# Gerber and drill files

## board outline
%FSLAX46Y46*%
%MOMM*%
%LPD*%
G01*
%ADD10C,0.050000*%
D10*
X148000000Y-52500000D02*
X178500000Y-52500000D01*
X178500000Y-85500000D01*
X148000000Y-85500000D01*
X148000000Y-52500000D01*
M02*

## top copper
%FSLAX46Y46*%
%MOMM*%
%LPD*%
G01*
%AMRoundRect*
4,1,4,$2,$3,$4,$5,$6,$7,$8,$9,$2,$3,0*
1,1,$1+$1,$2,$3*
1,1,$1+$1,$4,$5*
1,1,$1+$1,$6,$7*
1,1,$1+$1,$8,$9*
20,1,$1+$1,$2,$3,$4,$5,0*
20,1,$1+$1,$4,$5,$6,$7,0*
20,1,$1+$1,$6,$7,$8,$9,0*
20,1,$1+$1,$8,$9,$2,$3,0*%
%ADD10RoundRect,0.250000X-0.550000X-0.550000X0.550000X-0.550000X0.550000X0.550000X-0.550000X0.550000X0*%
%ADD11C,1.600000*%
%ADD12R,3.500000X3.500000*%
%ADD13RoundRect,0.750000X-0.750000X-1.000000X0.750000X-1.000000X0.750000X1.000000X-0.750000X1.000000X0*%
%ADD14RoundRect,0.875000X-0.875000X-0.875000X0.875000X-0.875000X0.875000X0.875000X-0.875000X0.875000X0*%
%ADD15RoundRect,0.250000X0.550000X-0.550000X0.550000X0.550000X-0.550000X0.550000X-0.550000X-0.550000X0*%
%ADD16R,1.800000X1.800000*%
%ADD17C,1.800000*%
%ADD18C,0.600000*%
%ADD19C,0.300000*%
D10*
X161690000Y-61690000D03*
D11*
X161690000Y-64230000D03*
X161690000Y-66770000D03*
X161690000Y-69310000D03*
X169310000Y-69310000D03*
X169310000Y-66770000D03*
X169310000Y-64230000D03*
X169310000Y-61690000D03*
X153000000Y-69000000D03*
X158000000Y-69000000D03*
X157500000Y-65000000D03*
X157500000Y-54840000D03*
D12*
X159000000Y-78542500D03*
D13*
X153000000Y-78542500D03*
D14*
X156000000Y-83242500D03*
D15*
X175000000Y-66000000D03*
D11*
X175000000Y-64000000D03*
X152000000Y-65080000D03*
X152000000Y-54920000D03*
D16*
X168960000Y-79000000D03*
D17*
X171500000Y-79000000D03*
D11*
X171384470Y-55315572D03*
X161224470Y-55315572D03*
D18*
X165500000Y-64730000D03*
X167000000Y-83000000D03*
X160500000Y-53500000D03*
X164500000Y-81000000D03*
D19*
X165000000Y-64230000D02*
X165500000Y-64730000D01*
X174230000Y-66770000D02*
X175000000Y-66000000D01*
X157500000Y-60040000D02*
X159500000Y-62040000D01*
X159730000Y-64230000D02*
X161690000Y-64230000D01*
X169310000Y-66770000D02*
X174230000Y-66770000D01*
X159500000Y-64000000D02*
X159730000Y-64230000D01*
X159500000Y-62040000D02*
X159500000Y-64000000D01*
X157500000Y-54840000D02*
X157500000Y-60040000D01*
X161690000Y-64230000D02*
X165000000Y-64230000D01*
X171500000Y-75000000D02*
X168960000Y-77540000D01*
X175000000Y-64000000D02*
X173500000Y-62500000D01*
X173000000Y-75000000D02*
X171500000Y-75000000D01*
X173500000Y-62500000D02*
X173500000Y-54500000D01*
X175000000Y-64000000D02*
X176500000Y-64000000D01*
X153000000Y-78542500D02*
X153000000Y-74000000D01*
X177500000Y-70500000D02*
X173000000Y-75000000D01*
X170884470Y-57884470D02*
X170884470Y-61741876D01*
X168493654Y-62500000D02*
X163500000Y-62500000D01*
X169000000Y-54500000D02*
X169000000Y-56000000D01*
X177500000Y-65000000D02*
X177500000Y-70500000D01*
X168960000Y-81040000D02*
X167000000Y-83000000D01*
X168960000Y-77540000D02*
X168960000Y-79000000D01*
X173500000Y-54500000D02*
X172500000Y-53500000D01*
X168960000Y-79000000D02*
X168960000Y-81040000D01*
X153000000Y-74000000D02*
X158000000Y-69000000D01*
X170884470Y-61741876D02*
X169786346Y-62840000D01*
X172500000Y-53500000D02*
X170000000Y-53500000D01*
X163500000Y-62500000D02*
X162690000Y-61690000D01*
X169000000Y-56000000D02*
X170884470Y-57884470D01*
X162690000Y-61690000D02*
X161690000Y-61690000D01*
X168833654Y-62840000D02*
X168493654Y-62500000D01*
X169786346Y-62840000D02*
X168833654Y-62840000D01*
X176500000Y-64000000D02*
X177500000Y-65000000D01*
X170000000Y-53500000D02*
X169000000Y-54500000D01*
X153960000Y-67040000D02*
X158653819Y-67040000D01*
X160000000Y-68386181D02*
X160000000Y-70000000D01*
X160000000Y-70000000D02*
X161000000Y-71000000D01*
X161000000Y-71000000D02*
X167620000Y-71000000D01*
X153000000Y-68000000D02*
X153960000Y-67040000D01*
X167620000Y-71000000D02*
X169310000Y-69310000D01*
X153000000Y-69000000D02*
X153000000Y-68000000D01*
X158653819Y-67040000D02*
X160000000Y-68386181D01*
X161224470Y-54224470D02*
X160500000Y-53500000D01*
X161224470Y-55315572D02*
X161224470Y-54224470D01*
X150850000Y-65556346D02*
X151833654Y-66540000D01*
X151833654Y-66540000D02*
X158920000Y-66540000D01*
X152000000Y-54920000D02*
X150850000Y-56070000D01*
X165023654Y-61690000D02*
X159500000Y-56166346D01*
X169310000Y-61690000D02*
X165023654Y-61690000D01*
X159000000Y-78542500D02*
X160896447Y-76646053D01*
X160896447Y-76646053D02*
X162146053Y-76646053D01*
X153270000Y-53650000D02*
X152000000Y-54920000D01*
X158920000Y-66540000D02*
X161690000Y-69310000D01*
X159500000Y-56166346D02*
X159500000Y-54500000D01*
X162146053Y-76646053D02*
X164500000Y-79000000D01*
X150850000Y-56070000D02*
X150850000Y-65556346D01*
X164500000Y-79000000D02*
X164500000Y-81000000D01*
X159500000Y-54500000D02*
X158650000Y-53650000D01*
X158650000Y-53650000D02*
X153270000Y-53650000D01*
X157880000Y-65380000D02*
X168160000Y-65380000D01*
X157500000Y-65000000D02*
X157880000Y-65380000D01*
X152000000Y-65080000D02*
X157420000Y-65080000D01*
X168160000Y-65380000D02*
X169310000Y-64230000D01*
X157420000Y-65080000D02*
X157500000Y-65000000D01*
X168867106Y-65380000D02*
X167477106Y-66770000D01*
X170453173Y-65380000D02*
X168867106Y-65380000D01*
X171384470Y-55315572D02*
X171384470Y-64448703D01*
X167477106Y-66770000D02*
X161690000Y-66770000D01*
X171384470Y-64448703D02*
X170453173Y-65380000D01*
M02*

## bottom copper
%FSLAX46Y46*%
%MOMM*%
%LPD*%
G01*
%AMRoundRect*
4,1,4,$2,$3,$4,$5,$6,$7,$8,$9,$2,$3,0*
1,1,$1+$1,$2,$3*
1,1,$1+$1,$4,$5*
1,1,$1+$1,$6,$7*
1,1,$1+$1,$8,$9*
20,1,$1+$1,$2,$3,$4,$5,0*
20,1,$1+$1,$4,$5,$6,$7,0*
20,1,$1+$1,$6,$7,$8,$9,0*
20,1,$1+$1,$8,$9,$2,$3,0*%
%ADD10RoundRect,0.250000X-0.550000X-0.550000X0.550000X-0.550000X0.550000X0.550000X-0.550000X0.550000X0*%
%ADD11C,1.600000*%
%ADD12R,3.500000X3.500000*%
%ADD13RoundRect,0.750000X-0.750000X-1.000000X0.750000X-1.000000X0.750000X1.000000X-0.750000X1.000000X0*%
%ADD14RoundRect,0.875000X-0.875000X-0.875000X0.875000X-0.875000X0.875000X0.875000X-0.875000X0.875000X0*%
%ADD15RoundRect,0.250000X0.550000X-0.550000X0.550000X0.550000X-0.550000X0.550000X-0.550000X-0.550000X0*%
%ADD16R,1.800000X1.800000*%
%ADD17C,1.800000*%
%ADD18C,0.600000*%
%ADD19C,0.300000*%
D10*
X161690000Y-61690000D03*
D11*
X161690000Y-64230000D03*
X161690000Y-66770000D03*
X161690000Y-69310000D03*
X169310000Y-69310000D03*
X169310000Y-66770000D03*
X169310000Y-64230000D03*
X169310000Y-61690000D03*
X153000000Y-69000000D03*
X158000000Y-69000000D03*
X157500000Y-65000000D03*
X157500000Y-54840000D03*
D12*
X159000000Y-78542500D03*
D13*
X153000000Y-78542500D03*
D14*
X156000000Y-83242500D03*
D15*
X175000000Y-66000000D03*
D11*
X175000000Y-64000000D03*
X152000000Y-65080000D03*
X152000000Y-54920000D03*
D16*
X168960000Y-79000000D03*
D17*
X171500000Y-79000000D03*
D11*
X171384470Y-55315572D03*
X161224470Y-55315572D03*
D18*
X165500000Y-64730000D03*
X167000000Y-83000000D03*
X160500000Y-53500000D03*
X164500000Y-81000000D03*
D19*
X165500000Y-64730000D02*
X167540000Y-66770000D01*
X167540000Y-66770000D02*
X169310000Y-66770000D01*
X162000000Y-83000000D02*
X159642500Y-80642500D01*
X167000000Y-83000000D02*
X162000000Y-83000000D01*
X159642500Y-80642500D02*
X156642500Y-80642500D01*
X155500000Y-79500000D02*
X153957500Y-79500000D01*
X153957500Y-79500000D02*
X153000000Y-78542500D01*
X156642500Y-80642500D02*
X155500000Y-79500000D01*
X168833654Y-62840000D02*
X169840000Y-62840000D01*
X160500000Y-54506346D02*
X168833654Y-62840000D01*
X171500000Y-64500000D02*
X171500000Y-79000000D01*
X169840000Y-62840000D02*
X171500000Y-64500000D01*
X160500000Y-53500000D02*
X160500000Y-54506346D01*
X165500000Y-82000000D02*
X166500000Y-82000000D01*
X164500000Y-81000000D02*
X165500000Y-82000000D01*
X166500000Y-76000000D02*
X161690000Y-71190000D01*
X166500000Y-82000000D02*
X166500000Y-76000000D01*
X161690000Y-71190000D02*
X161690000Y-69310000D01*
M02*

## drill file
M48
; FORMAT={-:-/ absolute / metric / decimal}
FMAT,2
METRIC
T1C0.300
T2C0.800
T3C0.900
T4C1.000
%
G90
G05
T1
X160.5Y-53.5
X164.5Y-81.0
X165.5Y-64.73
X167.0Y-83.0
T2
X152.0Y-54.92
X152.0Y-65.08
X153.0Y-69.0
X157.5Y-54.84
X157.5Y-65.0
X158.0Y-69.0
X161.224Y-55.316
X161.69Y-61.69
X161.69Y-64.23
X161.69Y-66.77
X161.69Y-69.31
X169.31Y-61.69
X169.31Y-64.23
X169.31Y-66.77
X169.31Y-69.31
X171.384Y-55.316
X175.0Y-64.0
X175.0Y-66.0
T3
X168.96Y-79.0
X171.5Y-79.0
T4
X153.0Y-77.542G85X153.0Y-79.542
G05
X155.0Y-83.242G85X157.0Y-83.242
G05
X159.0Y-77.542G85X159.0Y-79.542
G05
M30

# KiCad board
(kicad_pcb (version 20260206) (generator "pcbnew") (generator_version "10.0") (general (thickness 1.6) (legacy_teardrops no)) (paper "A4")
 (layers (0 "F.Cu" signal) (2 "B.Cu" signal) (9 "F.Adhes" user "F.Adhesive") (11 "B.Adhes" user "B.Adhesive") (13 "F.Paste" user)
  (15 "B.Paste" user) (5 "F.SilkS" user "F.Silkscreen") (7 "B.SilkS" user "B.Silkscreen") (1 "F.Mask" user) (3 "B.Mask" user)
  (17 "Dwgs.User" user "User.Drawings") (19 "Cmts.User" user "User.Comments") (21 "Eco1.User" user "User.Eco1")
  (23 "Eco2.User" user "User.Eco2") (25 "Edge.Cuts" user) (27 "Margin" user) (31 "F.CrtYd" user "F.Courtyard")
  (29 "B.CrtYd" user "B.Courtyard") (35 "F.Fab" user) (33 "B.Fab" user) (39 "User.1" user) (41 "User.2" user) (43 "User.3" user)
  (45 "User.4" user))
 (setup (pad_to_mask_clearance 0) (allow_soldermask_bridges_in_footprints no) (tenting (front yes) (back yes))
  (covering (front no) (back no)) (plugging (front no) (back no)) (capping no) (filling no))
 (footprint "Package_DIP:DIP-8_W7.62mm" (layer "F.Cu") (at 161.69 61.69)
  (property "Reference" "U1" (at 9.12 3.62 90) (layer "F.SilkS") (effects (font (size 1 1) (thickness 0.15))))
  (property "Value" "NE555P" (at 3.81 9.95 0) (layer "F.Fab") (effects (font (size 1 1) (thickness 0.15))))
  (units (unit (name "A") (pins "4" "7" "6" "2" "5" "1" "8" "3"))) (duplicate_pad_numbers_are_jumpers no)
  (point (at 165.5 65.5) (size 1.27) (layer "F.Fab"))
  (pad "1" thru_hole roundrect (at 0 0) (size 1.6 1.6) (drill 0.8) (layers "*.Cu" "*.Mask") (remove_unused_layers no)
   (roundrect_rratio 0.15625) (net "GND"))
  (pad "2" thru_hole circle (at 0 2.54) (size 1.6 1.6) (drill 0.8) (layers "*.Cu" "*.Mask") (remove_unused_layers no) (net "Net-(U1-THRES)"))
  (pad "3" thru_hole circle (at 0 5.08) (size 1.6 1.6) (drill 0.8) (layers "*.Cu" "*.Mask") (remove_unused_layers no) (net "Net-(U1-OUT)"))
  (pad "4" thru_hole circle (at 0 7.62) (size 1.6 1.6) (drill 0.8) (layers "*.Cu" "*.Mask") (remove_unused_layers no) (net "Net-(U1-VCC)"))
  (pad "5" thru_hole circle (at 7.62 7.62) (size 1.6 1.6) (drill 0.8) (layers "*.Cu" "*.Mask") (remove_unused_layers no)
   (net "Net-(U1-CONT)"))
  (pad "6" thru_hole circle (at 7.62 5.08) (size 1.6 1.6) (drill 0.8) (layers "*.Cu" "*.Mask") (remove_unused_layers no)
   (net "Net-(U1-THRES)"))
  (pad "7" thru_hole circle (at 7.62 2.54) (size 1.6 1.6) (drill 0.8) (layers "*.Cu" "*.Mask") (remove_unused_layers no)
   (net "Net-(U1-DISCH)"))
  (pad "8" thru_hole circle (at 7.62 0) (size 1.6 1.6) (drill 0.8) (layers "*.Cu" "*.Mask") (remove_unused_layers no) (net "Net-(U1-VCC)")))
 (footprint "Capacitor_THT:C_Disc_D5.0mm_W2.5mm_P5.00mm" (layer "F.Cu") (at 153 69)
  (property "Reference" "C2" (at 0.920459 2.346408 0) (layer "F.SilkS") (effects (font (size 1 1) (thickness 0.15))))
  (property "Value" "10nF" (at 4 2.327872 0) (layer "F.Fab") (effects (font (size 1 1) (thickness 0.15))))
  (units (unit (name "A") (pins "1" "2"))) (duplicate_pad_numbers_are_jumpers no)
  (pad "1" thru_hole circle (at 0 0) (size 1.6 1.6) (drill 0.8) (layers "*.Cu" "*.Mask") (remove_unused_layers no) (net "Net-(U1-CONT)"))
  (pad "2" thru_hole circle (at 5 0) (size 1.6 1.6) (drill 0.8) (layers "*.Cu" "*.Mask") (remove_unused_layers no) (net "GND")))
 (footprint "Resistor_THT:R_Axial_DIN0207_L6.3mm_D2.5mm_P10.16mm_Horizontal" (layer "F.Cu") (at 157.5 65 90)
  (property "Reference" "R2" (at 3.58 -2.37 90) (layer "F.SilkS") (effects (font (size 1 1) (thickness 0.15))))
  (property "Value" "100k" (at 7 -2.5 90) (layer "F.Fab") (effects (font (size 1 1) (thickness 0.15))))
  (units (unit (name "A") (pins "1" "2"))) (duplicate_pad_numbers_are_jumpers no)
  (pad "1" thru_hole circle (at 0 0 90) (size 1.6 1.6) (drill 0.8) (layers "*.Cu" "*.Mask") (remove_unused_layers no) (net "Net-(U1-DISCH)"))
  (pad "2" thru_hole circle (at 10.16 0 90) (size 1.6 1.6) (drill 0.8) (layers "*.Cu" "*.Mask") (remove_unused_layers no)
   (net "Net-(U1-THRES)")))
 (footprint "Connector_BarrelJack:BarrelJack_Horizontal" (layer "F.Cu") (at 159 78.5425)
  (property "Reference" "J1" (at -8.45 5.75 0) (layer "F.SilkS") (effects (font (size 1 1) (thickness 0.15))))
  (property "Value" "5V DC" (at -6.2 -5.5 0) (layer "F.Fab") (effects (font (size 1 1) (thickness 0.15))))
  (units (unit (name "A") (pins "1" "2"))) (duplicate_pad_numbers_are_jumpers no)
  (pad "1" thru_hole rect (at 0 0) (size 3.5 3.5) (drill oval 1 3) (layers "*.Cu" "*.Mask") (remove_unused_layers no) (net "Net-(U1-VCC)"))
  (pad "2" thru_hole roundrect (at -6 0) (size 3 3.5) (drill oval 1 3) (layers "*.Cu" "*.Mask") (remove_unused_layers no)
   (roundrect_rratio 0.25) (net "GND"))
  (pad "3" thru_hole roundrect (at -3 4.7) (size 3.5 3.5) (drill oval 3 1) (layers "*.Cu" "*.Mask") (remove_unused_layers no)
   (roundrect_rratio 0.25)))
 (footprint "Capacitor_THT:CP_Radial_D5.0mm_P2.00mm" (layer "F.Cu") (at 175 66 90)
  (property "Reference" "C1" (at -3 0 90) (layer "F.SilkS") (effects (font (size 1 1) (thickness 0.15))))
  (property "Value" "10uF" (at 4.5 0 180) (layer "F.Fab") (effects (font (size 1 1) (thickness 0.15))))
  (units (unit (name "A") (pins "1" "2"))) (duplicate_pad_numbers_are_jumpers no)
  (pad "1" thru_hole roundrect (at 0 0 90) (size 1.6 1.6) (drill 0.8) (layers "*.Cu" "*.Mask") (remove_unused_layers no)
   (roundrect_rratio 0.15625) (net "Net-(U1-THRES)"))
  (pad "2" thru_hole circle (at 2 0 90) (size 1.6 1.6) (drill 0.8) (layers "*.Cu" "*.Mask") (remove_unused_layers no) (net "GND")))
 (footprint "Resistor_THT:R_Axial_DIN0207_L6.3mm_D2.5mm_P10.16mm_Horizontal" (layer "F.Cu") (at 152 65.08 90)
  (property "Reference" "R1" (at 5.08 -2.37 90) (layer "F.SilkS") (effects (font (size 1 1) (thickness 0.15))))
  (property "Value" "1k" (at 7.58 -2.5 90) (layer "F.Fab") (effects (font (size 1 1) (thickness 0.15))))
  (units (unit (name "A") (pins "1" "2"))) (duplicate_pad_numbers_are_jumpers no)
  (pad "1" thru_hole circle (at 0 0 90) (size 1.6 1.6) (drill 0.8) (layers "*.Cu" "*.Mask") (remove_unused_layers no) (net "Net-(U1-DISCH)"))
  (pad "2" thru_hole circle (at 10.16 0 90) (size 1.6 1.6) (drill 0.8) (layers "*.Cu" "*.Mask") (remove_unused_layers no)
   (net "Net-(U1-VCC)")))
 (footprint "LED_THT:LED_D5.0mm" (layer "F.Cu") (at 168.96 79)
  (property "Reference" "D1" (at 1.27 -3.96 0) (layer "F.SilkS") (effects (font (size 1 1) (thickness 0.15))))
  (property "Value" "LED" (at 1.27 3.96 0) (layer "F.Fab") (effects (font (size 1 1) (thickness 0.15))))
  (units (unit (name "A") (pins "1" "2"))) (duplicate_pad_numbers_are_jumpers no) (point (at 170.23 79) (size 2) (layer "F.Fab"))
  (pad "1" thru_hole rect (at 0 0) (size 1.8 1.8) (drill 0.9) (layers "*.Cu" "*.Mask") (remove_unused_layers no) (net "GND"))
  (pad "2" thru_hole circle (at 2.54 0) (size 1.8 1.8) (drill 0.9) (layers "*.Cu" "*.Mask") (remove_unused_layers no) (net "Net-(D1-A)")))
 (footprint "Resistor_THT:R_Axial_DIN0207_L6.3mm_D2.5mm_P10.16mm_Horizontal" (layer "F.Cu") (at 171.38447 55.315572 180)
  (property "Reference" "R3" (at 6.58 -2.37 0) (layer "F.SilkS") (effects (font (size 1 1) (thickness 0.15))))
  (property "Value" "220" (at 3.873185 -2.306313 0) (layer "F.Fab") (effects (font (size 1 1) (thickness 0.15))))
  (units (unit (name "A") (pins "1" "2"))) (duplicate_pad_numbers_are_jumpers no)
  (pad "1" thru_hole circle (at 0 0 180) (size 1.6 1.6) (drill 0.8) (layers "*.Cu" "*.Mask") (remove_unused_layers no) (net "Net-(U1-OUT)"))
  (pad "2" thru_hole circle (at 10.16 0 180) (size 1.6 1.6) (drill 0.8) (layers "*.Cu" "*.Mask") (remove_unused_layers no)
   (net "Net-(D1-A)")))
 (gr_rect (start 148 52.5) (end 178.5 85.5) (stroke (width 0.05) (type default)) (fill no) (layer "Edge.Cuts"))
 (segment (start 165 64.23) (end 165.5 64.73) (width 0.3) (layer "F.Cu") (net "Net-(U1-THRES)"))
 (segment (start 174.23 66.77) (end 175 66) (width 0.3) (layer "F.Cu") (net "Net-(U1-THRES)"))
 (segment (start 157.5 60.04) (end 159.5 62.04) (width 0.3) (layer "F.Cu") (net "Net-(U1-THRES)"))
 (segment (start 159.73 64.23) (end 161.69 64.23) (width 0.3) (layer "F.Cu") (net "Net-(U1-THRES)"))
 (segment (start 169.31 66.77) (end 174.23 66.77) (width 0.3) (layer "F.Cu") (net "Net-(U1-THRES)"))
 (segment (start 159.5 64) (end 159.73 64.23) (width 0.3) (layer "F.Cu") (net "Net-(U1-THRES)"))
 (segment (start 159.5 62.04) (end 159.5 64) (width 0.3) (layer "F.Cu") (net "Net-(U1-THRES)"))
 (segment (start 157.5 54.84) (end 157.5 60.04) (width 0.3) (layer "F.Cu") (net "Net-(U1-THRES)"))
 (segment (start 161.69 64.23) (end 165 64.23) (width 0.3) (layer "F.Cu") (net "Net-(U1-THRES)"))
 (via (at 165.5 64.73) (size 0.6) (drill 0.3) (layers "F.Cu" "B.Cu") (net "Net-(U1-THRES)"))
 (segment (start 165.5 64.73) (end 167.54 66.77) (width 0.3) (layer "B.Cu") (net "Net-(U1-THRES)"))
 (segment (start 167.54 66.77) (end 169.31 66.77) (width 0.3) (layer "B.Cu") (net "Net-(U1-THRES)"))
 (segment (start 171.5 75) (end 168.96 77.54) (width 0.3) (layer "F.Cu") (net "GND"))
 (segment (start 175 64) (end 173.5 62.5) (width 0.3) (layer "F.Cu") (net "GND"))
 (segment (start 173 75) (end 171.5 75) (width 0.3) (layer "F.Cu") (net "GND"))
 (segment (start 173.5 62.5) (end 173.5 54.5) (width 0.3) (layer "F.Cu") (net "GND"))
 (segment (start 175 64) (end 176.5 64) (width 0.3) (layer "F.Cu") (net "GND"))
 (segment (start 153 78.5425) (end 153 74) (width 0.3) (layer "F.Cu") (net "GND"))
 (segment (start 177.5 70.5) (end 173 75) (width 0.3) (layer "F.Cu") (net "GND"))
 (segment (start 170.88447 57.88447) (end 170.88447 61.741876) (width 0.3) (layer "F.Cu") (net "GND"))
 (segment (start 168.493654 62.5) (end 163.5 62.5) (width 0.3) (layer "F.Cu") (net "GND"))
 (segment (start 169 54.5) (end 169 56) (width 0.3) (layer "F.Cu") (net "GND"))
 (segment (start 177.5 65) (end 177.5 70.5) (width 0.3) (layer "F.Cu") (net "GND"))
 (segment (start 168.96 81.04) (end 167 83) (width 0.3) (layer "F.Cu") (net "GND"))
 (segment (start 168.96 77.54) (end 168.96 79) (width 0.3) (layer "F.Cu") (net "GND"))
 (segment (start 173.5 54.5) (end 172.5 53.5) (width 0.3) (layer "F.Cu") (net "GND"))
 (segment (start 168.96 79) (end 168.96 81.04) (width 0.3) (layer "F.Cu") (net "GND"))
 (segment (start 153 74) (end 158 69) (width 0.3) (layer "F.Cu") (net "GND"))
 (segment (start 170.88447 61.741876) (end 169.786346 62.84) (width 0.3) (layer "F.Cu") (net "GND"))
 (segment (start 172.5 53.5) (end 170 53.5) (width 0.3) (layer "F.Cu") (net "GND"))
 (segment (start 163.5 62.5) (end 162.69 61.69) (width 0.3) (layer "F.Cu") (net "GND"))
 (segment (start 169 56) (end 170.88447 57.88447) (width 0.3) (layer "F.Cu") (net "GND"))
 (segment (start 162.69 61.69) (end 161.69 61.69) (width 0.3) (layer "F.Cu") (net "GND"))
 (segment (start 168.833654 62.84) (end 168.493654 62.5) (width 0.3) (layer "F.Cu") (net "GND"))
 (segment (start 169.786346 62.84) (end 168.833654 62.84) (width 0.3) (layer "F.Cu") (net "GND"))
 (segment (start 176.5 64) (end 177.5 65) (width 0.3) (layer "F.Cu") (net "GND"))
 (segment (start 170 53.5) (end 169 54.5) (width 0.3) (layer "F.Cu") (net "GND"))
 (via (at 167 83) (size 0.6) (drill 0.3) (layers "F.Cu" "B.Cu") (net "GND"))
 (segment (start 162 83) (end 159.6425 80.6425) (width 0.3) (layer "B.Cu") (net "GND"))
 (segment (start 167 83) (end 162 83) (width 0.3) (layer "B.Cu") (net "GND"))
 (segment (start 159.6425 80.6425) (end 156.6425 80.6425) (width 0.3) (layer "B.Cu") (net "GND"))
 (segment (start 155.5 79.5) (end 153.9575 79.5) (width 0.3) (layer "B.Cu") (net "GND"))
 (segment (start 153.9575 79.5) (end 153 78.5425) (width 0.3) (layer "B.Cu") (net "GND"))
 (segment (start 156.6425 80.6425) (end 155.5 79.5) (width 0.3) (layer "B.Cu") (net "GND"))
 (segment (start 153.96 67.04) (end 158.653819 67.04) (width 0.3) (layer "F.Cu") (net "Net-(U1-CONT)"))
 (segment (start 160 68.386181) (end 160 70) (width 0.3) (layer "F.Cu") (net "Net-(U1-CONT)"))
 (segment (start 160 70) (end 161 71) (width 0.3) (layer "F.Cu") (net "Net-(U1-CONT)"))
 (segment (start 161 71) (end 167.62 71) (width 0.3) (layer "F.Cu") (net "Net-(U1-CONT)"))
 (segment (start 153 68) (end 153.96 67.04) (width 0.3) (layer "F.Cu") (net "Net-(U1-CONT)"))
 (segment (start 167.62 71) (end 169.31 69.31) (width 0.3) (layer "F.Cu") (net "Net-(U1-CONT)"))
 (segment (start 153 69) (end 153 68) (width 0.3) (layer "F.Cu") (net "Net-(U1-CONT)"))
 (segment (start 158.653819 67.04) (end 160 68.386181) (width 0.3) (layer "F.Cu") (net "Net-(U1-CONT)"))
 (segment (start 161.22447 54.22447) (end 160.5 53.5) (width 0.3) (layer "F.Cu") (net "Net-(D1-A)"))
 (segment (start 161.22447 55.315572) (end 161.22447 54.22447) (width 0.3) (layer "F.Cu") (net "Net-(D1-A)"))
 (via (at 160.5 53.5) (size 0.6) (drill 0.3) (layers "F.Cu" "B.Cu") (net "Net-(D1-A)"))
 (segment (start 168.833654 62.84) (end 169.84 62.84) (width 0.3) (layer "B.Cu") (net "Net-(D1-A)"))
 (segment (start 160.5 54.506346) (end 168.833654 62.84) (width 0.3) (layer "B.Cu") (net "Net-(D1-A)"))
 (segment (start 171.5 64.5) (end 171.5 79) (width 0.3) (layer "B.Cu") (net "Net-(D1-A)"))
 (segment (start 169.84 62.84) (end 171.5 64.5) (width 0.3) (layer "B.Cu") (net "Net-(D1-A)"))
 (segment (start 160.5 53.5) (end 160.5 54.506346) (width 0.3) (layer "B.Cu") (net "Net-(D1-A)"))
 (segment (start 150.85 65.556346) (end 151.833654 66.54) (width 0.3) (layer "F.Cu") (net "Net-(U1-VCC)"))
 (segment (start 151.833654 66.54) (end 158.92 66.54) (width 0.3) (layer "F.Cu") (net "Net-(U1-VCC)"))
 (segment (start 152 54.92) (end 150.85 56.07) (width 0.3) (layer "F.Cu") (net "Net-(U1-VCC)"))
 (segment (start 165.023654 61.69) (end 159.5 56.166346) (width 0.3) (layer "F.Cu") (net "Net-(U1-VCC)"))
 (segment (start 169.31 61.69) (end 165.023654 61.69) (width 0.3) (layer "F.Cu") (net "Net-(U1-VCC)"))
 (segment (start 159 78.5425) (end 160.896447 76.646053) (width 0.3) (layer "F.Cu") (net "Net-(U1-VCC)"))
 (segment (start 160.896447 76.646053) (end 162.146053 76.646053) (width 0.3) (layer "F.Cu") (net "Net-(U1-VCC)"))
 (segment (start 153.27 53.65) (end 152 54.92) (width 0.3) (layer "F.Cu") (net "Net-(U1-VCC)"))
 (segment (start 158.92 66.54) (end 161.69 69.31) (width 0.3) (layer "F.Cu") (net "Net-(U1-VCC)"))
 (segment (start 159.5 56.166346) (end 159.5 54.5) (width 0.3) (layer "F.Cu") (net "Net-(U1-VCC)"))
 (segment (start 162.146053 76.646053) (end 164.5 79) (width 0.3) (layer "F.Cu") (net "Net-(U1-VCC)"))
 (segment (start 150.85 56.07) (end 150.85 65.556346) (width 0.3) (layer "F.Cu") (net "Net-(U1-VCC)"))
 (segment (start 164.5 79) (end 164.5 81) (width 0.3) (layer "F.Cu") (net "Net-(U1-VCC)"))
 (segment (start 159.5 54.5) (end 158.65 53.65) (width 0.3) (layer "F.Cu") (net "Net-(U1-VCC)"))
 (segment (start 158.65 53.65) (end 153.27 53.65) (width 0.3) (layer "F.Cu") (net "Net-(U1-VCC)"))
 (via (at 164.5 81) (size 0.6) (drill 0.3) (layers "F.Cu" "B.Cu") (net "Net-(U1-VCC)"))
 (segment (start 165.5 82) (end 166.5 82) (width 0.3) (layer "B.Cu") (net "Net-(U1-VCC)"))
 (segment (start 164.5 81) (end 165.5 82) (width 0.3) (layer "B.Cu") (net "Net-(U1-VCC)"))
 (segment (start 166.5 76) (end 161.69 71.19) (width 0.3) (layer "B.Cu") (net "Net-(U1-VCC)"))
 (segment (start 166.5 82) (end 166.5 76) (width 0.3) (layer "B.Cu") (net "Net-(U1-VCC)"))
 (segment (start 161.69 71.19) (end 161.69 69.31) (width 0.3) (layer "B.Cu") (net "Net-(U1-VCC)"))
 (segment (start 157.88 65.38) (end 168.16 65.38) (width 0.3) (layer "F.Cu") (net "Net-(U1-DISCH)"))
 (segment (start 157.5 65) (end 157.88 65.38) (width 0.3) (layer "F.Cu") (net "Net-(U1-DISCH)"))
 (segment (start 152 65.08) (end 157.42 65.08) (width 0.3) (layer "F.Cu") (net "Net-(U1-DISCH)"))
 (segment (start 168.16 65.38) (end 169.31 64.23) (width 0.3) (layer "F.Cu") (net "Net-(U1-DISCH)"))
 (segment (start 157.42 65.08) (end 157.5 65) (width 0.3) (layer "F.Cu") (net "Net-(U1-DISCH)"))
 (segment (start 168.867106 65.38) (end 167.477106 66.77) (width 0.3) (layer "F.Cu") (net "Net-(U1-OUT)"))
 (segment (start 170.453173 65.38) (end 168.867106 65.38) (width 0.3) (layer "F.Cu") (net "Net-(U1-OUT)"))
 (segment (start 171.38447 55.315572) (end 171.38447 64.448703) (width 0.3) (layer "F.Cu") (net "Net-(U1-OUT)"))
 (segment (start 167.477106 66.77) (end 161.69 66.77) (width 0.3) (layer "F.Cu") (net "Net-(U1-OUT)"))
 (segment (start 171.38447 64.448703) (end 170.453173 65.38) (width 0.3) (layer "F.Cu") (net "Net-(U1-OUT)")))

